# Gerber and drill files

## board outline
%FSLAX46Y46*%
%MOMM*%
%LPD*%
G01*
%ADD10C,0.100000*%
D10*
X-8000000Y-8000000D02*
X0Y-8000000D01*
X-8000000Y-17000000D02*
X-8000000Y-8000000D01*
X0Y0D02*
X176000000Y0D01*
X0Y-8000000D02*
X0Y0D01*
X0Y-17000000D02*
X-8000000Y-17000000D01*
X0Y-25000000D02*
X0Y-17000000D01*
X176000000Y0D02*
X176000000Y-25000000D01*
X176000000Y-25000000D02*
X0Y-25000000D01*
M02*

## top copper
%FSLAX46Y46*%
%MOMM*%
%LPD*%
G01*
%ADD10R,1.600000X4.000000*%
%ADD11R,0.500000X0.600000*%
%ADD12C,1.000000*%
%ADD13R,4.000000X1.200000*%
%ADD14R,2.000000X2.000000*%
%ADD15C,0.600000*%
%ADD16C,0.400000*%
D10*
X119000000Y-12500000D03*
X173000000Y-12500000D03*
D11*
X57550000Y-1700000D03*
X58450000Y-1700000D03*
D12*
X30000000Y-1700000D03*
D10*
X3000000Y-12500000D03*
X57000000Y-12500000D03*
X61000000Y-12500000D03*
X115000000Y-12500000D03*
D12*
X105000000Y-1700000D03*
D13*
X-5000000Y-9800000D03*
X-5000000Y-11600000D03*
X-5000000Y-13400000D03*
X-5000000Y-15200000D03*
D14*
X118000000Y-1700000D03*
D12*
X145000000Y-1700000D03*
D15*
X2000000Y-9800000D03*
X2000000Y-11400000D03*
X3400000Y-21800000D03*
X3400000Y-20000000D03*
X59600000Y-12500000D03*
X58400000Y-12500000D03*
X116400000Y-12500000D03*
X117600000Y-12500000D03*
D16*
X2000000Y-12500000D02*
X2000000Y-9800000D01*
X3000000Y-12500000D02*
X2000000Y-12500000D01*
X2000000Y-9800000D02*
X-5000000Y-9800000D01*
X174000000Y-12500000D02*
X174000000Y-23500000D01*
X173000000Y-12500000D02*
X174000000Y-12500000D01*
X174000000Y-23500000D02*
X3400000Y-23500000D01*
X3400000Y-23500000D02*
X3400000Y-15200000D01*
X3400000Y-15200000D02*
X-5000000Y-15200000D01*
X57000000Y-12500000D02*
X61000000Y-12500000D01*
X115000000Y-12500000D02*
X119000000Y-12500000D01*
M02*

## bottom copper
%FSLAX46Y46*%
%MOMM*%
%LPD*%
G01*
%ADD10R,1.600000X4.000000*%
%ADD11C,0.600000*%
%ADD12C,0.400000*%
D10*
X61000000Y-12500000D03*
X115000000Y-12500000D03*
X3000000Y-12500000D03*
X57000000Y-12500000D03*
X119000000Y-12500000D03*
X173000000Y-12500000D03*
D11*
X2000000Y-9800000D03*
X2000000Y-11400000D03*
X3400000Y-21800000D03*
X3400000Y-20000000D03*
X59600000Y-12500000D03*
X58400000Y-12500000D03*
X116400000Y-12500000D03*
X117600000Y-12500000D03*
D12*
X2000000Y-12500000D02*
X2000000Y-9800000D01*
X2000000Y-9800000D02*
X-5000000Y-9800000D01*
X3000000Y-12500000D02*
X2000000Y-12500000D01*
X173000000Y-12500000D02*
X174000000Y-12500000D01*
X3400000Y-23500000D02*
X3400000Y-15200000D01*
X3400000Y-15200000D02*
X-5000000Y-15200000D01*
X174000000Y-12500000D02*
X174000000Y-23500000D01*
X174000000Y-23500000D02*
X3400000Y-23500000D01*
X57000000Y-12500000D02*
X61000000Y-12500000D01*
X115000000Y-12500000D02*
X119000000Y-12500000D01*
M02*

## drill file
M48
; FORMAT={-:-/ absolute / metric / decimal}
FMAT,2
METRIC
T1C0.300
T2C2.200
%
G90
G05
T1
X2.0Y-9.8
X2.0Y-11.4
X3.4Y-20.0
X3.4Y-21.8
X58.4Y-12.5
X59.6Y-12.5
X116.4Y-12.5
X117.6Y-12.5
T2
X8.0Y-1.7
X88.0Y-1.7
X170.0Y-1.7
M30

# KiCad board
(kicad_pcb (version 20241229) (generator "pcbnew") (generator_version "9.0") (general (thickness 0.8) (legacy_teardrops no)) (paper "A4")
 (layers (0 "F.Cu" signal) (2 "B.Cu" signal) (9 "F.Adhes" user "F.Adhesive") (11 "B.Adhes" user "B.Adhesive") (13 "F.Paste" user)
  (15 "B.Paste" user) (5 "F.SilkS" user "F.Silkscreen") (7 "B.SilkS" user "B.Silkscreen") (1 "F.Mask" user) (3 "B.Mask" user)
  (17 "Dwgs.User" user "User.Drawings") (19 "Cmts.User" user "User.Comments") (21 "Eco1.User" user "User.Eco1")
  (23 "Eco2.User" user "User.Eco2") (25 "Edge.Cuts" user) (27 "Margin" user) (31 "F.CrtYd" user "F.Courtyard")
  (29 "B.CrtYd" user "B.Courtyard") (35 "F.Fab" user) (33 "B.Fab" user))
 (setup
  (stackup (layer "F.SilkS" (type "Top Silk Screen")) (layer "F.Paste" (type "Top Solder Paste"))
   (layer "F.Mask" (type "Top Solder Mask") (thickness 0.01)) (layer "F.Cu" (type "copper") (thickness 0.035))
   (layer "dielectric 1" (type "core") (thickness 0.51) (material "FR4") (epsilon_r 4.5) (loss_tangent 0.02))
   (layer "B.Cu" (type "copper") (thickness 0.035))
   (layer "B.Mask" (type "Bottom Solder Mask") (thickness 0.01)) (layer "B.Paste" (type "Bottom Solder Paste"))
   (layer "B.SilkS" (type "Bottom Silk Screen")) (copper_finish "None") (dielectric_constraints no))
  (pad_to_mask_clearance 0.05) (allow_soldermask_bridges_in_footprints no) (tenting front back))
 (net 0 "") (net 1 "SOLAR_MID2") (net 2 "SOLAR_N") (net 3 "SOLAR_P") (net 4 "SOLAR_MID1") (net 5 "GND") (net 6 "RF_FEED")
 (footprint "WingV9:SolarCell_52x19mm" (layer "F.Cu") (at 146 12.5)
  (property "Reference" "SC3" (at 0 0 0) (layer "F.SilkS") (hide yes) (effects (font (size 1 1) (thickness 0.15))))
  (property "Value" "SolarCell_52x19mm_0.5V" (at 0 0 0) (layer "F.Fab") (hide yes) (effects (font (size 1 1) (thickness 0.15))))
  (pad "1" smd rect (at -27 0) (size 1.6 4) (layers "F.Cu" "F.Mask" "F.Paste") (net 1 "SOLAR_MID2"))
  (pad "2" smd rect (at 27 0) (size 1.6 4) (layers "F.Cu" "F.Mask" "F.Paste") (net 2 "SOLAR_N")))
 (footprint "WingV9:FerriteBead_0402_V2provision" (layer "F.Cu") (at 58 1.7)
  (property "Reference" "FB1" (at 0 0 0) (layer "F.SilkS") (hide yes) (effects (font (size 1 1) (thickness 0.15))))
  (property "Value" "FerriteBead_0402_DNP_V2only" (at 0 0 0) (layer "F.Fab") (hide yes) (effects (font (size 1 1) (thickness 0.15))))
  (pad "1" smd rect (at -0.45 0) (size 0.5 0.6) (layers "F.Cu" "F.Mask" "F.Paste"))
  (pad "2" smd rect (at 0.45 0) (size 0.5 0.6) (layers "F.Cu" "F.Mask" "F.Paste")))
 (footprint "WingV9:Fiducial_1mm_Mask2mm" (layer "F.Cu") (at 30 1.7)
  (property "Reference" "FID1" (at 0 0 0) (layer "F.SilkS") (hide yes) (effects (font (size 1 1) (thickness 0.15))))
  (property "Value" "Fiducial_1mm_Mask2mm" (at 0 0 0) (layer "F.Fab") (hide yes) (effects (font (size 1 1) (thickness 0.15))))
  (pad "1" smd circle (at 0 0) (size 1 1) (layers "F.Cu" "F.Mask")))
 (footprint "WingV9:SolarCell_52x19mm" (layer "F.Cu") (at 30 12.5)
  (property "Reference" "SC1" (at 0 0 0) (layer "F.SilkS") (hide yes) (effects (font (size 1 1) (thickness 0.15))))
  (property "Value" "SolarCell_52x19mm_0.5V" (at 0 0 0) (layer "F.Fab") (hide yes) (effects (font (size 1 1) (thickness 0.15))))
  (pad "1" smd rect (at -27 0) (size 1.6 4) (layers "F.Cu" "F.Mask" "F.Paste") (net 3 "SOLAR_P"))
  (pad "2" smd rect (at 27 0) (size 1.6 4) (layers "F.Cu" "F.Mask" "F.Paste") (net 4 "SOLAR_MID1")))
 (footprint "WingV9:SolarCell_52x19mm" (layer "F.Cu") (at 88 12.5)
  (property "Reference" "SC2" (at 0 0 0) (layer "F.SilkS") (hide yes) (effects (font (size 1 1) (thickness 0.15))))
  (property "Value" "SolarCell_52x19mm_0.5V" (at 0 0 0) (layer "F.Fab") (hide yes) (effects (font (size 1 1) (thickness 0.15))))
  (pad "1" smd rect (at -27 0) (size 1.6 4) (layers "F.Cu" "F.Mask" "F.Paste") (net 4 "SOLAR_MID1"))
  (pad "2" smd rect (at 27 0) (size 1.6 4) (layers "F.Cu" "F.Mask" "F.Paste") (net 1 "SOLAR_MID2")))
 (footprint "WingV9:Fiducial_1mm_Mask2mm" (layer "F.Cu") (at 105 1.7)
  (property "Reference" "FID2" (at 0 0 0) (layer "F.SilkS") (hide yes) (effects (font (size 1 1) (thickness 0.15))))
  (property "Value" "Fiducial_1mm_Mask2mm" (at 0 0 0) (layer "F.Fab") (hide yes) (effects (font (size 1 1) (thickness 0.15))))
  (pad "1" smd circle (at 0 0) (size 1 1) (layers "F.Cu" "F.Mask")))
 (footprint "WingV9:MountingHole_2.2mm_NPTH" (layer "F.Cu") (at 8 1.7)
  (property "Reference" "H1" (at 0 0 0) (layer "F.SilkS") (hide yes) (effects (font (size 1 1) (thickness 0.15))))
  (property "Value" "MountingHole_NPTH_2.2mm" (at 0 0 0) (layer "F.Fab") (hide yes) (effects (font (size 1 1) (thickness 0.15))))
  (pad "" np_thru_hole circle (at 0 0) (size 2.2 2.2) (drill 2.2) (layers "*.Cu" "*.Mask")))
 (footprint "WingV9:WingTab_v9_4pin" (layer "F.Cu") (at 0 0)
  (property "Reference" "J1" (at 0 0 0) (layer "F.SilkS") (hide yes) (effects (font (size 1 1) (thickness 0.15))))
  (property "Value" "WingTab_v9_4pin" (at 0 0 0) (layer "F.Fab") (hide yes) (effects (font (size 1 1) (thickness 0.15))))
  (pad "1" smd rect (at -5 9.8) (size 4 1.2) (layers "F.Cu" "F.Mask" "F.Paste") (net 3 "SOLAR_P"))
  (pad "2" smd rect (at -5 11.6) (size 4 1.2) (layers "F.Cu" "F.Mask" "F.Paste") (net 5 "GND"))
  (pad "3" smd rect (at -5 13.4) (size 4 1.2) (layers "F.Cu" "F.Mask" "F.Paste") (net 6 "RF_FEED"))
  (pad "4" smd rect (at -5 15.2) (size 4 1.2) (layers "F.Cu" "F.Mask" "F.Paste") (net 2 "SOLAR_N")))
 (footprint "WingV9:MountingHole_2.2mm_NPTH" (layer "F.Cu") (at 170 1.7)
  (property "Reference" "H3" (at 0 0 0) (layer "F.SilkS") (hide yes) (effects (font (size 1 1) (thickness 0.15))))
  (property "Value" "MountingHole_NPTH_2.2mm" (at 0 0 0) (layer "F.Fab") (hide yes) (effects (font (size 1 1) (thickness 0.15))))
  (pad "" np_thru_hole circle (at 0 0) (size 2.2 2.2) (drill 2.2) (layers "*.Cu" "*.Mask")))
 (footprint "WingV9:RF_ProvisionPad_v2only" (layer "F.Cu") (at 118 1.7)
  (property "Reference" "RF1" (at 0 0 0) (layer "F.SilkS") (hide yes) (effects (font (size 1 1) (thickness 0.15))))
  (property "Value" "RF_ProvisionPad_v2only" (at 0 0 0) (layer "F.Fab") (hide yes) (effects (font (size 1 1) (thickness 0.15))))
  (pad "1" smd rect (at 0 0) (size 2 2) (layers "F.Cu" "F.Mask")))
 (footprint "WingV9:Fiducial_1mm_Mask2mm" (layer "F.Cu") (at 145 1.7)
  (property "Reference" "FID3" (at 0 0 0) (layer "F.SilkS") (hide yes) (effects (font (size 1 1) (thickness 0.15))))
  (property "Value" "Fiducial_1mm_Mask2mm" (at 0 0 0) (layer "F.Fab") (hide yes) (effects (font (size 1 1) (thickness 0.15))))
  (pad "1" smd circle (at 0 0) (size 1 1) (layers "F.Cu" "F.Mask")))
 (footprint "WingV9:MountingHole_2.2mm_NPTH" (layer "F.Cu") (at 88 1.7)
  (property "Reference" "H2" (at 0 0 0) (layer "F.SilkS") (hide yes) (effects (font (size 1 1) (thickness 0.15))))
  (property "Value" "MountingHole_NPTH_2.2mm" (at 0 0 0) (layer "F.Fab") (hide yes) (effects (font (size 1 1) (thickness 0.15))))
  (pad "" np_thru_hole circle (at 0 0) (size 2.2 2.2) (drill 2.2) (layers "*.Cu" "*.Mask")))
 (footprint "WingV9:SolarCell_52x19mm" (layer "B.Cu") (at 88 12.5)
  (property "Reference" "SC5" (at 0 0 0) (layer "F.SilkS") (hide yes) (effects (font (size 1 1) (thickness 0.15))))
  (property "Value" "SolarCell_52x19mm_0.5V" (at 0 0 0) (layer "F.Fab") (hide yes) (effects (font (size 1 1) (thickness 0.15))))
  (pad "1" smd rect (at -27 0) (size 1.6 4) (layers "B.Cu" "B.Mask" "B.Paste") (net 4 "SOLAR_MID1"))
  (pad "2" smd rect (at 27 0) (size 1.6 4) (layers "B.Cu" "B.Mask" "B.Paste") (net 1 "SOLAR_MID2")))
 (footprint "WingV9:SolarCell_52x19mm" (layer "B.Cu") (at 30 12.5)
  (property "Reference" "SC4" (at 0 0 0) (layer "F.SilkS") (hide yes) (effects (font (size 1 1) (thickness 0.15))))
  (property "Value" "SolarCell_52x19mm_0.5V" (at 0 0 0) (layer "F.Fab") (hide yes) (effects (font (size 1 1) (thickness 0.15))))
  (pad "1" smd rect (at -27 0) (size 1.6 4) (layers "B.Cu" "B.Mask" "B.Paste") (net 3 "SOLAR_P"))
  (pad "2" smd rect (at 27 0) (size 1.6 4) (layers "B.Cu" "B.Mask" "B.Paste") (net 4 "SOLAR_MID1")))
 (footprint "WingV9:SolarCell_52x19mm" (layer "B.Cu") (at 146 12.5)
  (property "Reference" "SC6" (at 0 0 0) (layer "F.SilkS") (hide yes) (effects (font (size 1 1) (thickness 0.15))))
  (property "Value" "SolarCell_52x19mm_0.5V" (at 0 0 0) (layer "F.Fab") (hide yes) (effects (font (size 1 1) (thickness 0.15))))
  (pad "1" smd rect (at -27 0) (size 1.6 4) (layers "B.Cu" "B.Mask" "B.Paste") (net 1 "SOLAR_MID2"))
  (pad "2" smd rect (at 27 0) (size 1.6 4) (layers "B.Cu" "B.Mask" "B.Paste") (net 2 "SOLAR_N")))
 (gr_line (start -8 8) (end 0 8) (stroke (width 0.1) (type default)) (layer "Edge.Cuts"))
 (gr_line (start -8 17) (end -8 8) (stroke (width 0.1) (type default)) (layer "Edge.Cuts"))
 (gr_line (start 0 0) (end 176 0) (stroke (width 0.1) (type default)) (layer "Edge.Cuts"))
 (gr_line (start 0 8) (end 0 0) (stroke (width 0.1) (type default)) (layer "Edge.Cuts"))
 (gr_line (start 0 17) (end -8 17) (stroke (width 0.1) (type default)) (layer "Edge.Cuts"))
 (gr_line (start 0 25) (end 0 17) (stroke (width 0.1) (type default)) (layer "Edge.Cuts"))
 (gr_line (start 176 0) (end 176 25) (stroke (width 0.1) (type default)) (layer "Edge.Cuts"))
 (gr_line (start 176 25) (end 0 25) (stroke (width 0.1) (type default)) (layer "Edge.Cuts"))
 (segment (start 2 12.5) (end 2 9.8) (width 0.4) (layer "F.Cu") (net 3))
 (segment (start 3 12.5) (end 2 12.5) (width 0.4) (layer "F.Cu") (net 3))
 (segment (start 2 9.8) (end -5 9.8) (width 0.4) (layer "F.Cu") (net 3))
 (via (at 2 9.8) (size 0.6) (drill 0.3) (layers "F.Cu" "B.Cu") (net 3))
 (via (at 2 11.4) (size 0.6) (drill 0.3) (layers "F.Cu" "B.Cu") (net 3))
 (segment (start 2 12.5) (end 2 9.8) (width 0.4) (layer "B.Cu") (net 3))
 (segment (start 2 9.8) (end -5 9.8) (width 0.4) (layer "B.Cu") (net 3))
 (segment (start 3 12.5) (end 2 12.5) (width 0.4) (layer "B.Cu") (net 3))
 (segment (start 174 12.5) (end 174 23.5) (width 0.4) (layer "F.Cu") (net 2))
 (segment (start 173 12.5) (end 174 12.5) (width 0.4) (layer "F.Cu") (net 2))
 (segment (start 174 23.5) (end 3.4 23.5) (width 0.4) (layer "F.Cu") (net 2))
 (segment (start 3.4 23.5) (end 3.4 15.2) (width 0.4) (layer "F.Cu") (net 2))
 (segment (start 3.4 15.2) (end -5 15.2) (width 0.4) (layer "F.Cu") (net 2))
 (via (at 3.4 21.8) (size 0.6) (drill 0.3) (layers "F.Cu" "B.Cu") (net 2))
 (via (at 3.4 20) (size 0.6) (drill 0.3) (layers "F.Cu" "B.Cu") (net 2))
 (segment (start 173 12.5) (end 174 12.5) (width 0.4) (layer "B.Cu") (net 2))
 (segment (start 3.4 23.5) (end 3.4 15.2) (width 0.4) (layer "B.Cu") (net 2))
 (segment (start 3.4 15.2) (end -5 15.2) (width 0.4) (layer "B.Cu") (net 2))
 (segment (start 174 12.5) (end 174 23.5) (width 0.4) (layer "B.Cu") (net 2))
 (segment (start 174 23.5) (end 3.4 23.5) (width 0.4) (layer "B.Cu") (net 2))
 (segment (start 57 12.5) (end 61 12.5) (width 0.4) (layer "F.Cu") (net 4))
 (via (at 59.6 12.5) (size 0.6) (drill 0.3) (layers "F.Cu" "B.Cu") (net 4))
 (via (at 58.4 12.5) (size 0.6) (drill 0.3) (layers "F.Cu" "B.Cu") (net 4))
 (segment (start 57 12.5) (end 61 12.5) (width 0.4) (layer "B.Cu") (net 4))
 (segment (start 115 12.5) (end 119 12.5) (width 0.4) (layer "F.Cu") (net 1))
 (via (at 116.4 12.5) (size 0.6) (drill 0.3) (layers "F.Cu" "B.Cu") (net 1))
 (via (at 117.6 12.5) (size 0.6) (drill 0.3) (layers "F.Cu" "B.Cu") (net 1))
 (segment (start 115 12.5) (end 119 12.5) (width 0.4) (layer "B.Cu") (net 1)))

